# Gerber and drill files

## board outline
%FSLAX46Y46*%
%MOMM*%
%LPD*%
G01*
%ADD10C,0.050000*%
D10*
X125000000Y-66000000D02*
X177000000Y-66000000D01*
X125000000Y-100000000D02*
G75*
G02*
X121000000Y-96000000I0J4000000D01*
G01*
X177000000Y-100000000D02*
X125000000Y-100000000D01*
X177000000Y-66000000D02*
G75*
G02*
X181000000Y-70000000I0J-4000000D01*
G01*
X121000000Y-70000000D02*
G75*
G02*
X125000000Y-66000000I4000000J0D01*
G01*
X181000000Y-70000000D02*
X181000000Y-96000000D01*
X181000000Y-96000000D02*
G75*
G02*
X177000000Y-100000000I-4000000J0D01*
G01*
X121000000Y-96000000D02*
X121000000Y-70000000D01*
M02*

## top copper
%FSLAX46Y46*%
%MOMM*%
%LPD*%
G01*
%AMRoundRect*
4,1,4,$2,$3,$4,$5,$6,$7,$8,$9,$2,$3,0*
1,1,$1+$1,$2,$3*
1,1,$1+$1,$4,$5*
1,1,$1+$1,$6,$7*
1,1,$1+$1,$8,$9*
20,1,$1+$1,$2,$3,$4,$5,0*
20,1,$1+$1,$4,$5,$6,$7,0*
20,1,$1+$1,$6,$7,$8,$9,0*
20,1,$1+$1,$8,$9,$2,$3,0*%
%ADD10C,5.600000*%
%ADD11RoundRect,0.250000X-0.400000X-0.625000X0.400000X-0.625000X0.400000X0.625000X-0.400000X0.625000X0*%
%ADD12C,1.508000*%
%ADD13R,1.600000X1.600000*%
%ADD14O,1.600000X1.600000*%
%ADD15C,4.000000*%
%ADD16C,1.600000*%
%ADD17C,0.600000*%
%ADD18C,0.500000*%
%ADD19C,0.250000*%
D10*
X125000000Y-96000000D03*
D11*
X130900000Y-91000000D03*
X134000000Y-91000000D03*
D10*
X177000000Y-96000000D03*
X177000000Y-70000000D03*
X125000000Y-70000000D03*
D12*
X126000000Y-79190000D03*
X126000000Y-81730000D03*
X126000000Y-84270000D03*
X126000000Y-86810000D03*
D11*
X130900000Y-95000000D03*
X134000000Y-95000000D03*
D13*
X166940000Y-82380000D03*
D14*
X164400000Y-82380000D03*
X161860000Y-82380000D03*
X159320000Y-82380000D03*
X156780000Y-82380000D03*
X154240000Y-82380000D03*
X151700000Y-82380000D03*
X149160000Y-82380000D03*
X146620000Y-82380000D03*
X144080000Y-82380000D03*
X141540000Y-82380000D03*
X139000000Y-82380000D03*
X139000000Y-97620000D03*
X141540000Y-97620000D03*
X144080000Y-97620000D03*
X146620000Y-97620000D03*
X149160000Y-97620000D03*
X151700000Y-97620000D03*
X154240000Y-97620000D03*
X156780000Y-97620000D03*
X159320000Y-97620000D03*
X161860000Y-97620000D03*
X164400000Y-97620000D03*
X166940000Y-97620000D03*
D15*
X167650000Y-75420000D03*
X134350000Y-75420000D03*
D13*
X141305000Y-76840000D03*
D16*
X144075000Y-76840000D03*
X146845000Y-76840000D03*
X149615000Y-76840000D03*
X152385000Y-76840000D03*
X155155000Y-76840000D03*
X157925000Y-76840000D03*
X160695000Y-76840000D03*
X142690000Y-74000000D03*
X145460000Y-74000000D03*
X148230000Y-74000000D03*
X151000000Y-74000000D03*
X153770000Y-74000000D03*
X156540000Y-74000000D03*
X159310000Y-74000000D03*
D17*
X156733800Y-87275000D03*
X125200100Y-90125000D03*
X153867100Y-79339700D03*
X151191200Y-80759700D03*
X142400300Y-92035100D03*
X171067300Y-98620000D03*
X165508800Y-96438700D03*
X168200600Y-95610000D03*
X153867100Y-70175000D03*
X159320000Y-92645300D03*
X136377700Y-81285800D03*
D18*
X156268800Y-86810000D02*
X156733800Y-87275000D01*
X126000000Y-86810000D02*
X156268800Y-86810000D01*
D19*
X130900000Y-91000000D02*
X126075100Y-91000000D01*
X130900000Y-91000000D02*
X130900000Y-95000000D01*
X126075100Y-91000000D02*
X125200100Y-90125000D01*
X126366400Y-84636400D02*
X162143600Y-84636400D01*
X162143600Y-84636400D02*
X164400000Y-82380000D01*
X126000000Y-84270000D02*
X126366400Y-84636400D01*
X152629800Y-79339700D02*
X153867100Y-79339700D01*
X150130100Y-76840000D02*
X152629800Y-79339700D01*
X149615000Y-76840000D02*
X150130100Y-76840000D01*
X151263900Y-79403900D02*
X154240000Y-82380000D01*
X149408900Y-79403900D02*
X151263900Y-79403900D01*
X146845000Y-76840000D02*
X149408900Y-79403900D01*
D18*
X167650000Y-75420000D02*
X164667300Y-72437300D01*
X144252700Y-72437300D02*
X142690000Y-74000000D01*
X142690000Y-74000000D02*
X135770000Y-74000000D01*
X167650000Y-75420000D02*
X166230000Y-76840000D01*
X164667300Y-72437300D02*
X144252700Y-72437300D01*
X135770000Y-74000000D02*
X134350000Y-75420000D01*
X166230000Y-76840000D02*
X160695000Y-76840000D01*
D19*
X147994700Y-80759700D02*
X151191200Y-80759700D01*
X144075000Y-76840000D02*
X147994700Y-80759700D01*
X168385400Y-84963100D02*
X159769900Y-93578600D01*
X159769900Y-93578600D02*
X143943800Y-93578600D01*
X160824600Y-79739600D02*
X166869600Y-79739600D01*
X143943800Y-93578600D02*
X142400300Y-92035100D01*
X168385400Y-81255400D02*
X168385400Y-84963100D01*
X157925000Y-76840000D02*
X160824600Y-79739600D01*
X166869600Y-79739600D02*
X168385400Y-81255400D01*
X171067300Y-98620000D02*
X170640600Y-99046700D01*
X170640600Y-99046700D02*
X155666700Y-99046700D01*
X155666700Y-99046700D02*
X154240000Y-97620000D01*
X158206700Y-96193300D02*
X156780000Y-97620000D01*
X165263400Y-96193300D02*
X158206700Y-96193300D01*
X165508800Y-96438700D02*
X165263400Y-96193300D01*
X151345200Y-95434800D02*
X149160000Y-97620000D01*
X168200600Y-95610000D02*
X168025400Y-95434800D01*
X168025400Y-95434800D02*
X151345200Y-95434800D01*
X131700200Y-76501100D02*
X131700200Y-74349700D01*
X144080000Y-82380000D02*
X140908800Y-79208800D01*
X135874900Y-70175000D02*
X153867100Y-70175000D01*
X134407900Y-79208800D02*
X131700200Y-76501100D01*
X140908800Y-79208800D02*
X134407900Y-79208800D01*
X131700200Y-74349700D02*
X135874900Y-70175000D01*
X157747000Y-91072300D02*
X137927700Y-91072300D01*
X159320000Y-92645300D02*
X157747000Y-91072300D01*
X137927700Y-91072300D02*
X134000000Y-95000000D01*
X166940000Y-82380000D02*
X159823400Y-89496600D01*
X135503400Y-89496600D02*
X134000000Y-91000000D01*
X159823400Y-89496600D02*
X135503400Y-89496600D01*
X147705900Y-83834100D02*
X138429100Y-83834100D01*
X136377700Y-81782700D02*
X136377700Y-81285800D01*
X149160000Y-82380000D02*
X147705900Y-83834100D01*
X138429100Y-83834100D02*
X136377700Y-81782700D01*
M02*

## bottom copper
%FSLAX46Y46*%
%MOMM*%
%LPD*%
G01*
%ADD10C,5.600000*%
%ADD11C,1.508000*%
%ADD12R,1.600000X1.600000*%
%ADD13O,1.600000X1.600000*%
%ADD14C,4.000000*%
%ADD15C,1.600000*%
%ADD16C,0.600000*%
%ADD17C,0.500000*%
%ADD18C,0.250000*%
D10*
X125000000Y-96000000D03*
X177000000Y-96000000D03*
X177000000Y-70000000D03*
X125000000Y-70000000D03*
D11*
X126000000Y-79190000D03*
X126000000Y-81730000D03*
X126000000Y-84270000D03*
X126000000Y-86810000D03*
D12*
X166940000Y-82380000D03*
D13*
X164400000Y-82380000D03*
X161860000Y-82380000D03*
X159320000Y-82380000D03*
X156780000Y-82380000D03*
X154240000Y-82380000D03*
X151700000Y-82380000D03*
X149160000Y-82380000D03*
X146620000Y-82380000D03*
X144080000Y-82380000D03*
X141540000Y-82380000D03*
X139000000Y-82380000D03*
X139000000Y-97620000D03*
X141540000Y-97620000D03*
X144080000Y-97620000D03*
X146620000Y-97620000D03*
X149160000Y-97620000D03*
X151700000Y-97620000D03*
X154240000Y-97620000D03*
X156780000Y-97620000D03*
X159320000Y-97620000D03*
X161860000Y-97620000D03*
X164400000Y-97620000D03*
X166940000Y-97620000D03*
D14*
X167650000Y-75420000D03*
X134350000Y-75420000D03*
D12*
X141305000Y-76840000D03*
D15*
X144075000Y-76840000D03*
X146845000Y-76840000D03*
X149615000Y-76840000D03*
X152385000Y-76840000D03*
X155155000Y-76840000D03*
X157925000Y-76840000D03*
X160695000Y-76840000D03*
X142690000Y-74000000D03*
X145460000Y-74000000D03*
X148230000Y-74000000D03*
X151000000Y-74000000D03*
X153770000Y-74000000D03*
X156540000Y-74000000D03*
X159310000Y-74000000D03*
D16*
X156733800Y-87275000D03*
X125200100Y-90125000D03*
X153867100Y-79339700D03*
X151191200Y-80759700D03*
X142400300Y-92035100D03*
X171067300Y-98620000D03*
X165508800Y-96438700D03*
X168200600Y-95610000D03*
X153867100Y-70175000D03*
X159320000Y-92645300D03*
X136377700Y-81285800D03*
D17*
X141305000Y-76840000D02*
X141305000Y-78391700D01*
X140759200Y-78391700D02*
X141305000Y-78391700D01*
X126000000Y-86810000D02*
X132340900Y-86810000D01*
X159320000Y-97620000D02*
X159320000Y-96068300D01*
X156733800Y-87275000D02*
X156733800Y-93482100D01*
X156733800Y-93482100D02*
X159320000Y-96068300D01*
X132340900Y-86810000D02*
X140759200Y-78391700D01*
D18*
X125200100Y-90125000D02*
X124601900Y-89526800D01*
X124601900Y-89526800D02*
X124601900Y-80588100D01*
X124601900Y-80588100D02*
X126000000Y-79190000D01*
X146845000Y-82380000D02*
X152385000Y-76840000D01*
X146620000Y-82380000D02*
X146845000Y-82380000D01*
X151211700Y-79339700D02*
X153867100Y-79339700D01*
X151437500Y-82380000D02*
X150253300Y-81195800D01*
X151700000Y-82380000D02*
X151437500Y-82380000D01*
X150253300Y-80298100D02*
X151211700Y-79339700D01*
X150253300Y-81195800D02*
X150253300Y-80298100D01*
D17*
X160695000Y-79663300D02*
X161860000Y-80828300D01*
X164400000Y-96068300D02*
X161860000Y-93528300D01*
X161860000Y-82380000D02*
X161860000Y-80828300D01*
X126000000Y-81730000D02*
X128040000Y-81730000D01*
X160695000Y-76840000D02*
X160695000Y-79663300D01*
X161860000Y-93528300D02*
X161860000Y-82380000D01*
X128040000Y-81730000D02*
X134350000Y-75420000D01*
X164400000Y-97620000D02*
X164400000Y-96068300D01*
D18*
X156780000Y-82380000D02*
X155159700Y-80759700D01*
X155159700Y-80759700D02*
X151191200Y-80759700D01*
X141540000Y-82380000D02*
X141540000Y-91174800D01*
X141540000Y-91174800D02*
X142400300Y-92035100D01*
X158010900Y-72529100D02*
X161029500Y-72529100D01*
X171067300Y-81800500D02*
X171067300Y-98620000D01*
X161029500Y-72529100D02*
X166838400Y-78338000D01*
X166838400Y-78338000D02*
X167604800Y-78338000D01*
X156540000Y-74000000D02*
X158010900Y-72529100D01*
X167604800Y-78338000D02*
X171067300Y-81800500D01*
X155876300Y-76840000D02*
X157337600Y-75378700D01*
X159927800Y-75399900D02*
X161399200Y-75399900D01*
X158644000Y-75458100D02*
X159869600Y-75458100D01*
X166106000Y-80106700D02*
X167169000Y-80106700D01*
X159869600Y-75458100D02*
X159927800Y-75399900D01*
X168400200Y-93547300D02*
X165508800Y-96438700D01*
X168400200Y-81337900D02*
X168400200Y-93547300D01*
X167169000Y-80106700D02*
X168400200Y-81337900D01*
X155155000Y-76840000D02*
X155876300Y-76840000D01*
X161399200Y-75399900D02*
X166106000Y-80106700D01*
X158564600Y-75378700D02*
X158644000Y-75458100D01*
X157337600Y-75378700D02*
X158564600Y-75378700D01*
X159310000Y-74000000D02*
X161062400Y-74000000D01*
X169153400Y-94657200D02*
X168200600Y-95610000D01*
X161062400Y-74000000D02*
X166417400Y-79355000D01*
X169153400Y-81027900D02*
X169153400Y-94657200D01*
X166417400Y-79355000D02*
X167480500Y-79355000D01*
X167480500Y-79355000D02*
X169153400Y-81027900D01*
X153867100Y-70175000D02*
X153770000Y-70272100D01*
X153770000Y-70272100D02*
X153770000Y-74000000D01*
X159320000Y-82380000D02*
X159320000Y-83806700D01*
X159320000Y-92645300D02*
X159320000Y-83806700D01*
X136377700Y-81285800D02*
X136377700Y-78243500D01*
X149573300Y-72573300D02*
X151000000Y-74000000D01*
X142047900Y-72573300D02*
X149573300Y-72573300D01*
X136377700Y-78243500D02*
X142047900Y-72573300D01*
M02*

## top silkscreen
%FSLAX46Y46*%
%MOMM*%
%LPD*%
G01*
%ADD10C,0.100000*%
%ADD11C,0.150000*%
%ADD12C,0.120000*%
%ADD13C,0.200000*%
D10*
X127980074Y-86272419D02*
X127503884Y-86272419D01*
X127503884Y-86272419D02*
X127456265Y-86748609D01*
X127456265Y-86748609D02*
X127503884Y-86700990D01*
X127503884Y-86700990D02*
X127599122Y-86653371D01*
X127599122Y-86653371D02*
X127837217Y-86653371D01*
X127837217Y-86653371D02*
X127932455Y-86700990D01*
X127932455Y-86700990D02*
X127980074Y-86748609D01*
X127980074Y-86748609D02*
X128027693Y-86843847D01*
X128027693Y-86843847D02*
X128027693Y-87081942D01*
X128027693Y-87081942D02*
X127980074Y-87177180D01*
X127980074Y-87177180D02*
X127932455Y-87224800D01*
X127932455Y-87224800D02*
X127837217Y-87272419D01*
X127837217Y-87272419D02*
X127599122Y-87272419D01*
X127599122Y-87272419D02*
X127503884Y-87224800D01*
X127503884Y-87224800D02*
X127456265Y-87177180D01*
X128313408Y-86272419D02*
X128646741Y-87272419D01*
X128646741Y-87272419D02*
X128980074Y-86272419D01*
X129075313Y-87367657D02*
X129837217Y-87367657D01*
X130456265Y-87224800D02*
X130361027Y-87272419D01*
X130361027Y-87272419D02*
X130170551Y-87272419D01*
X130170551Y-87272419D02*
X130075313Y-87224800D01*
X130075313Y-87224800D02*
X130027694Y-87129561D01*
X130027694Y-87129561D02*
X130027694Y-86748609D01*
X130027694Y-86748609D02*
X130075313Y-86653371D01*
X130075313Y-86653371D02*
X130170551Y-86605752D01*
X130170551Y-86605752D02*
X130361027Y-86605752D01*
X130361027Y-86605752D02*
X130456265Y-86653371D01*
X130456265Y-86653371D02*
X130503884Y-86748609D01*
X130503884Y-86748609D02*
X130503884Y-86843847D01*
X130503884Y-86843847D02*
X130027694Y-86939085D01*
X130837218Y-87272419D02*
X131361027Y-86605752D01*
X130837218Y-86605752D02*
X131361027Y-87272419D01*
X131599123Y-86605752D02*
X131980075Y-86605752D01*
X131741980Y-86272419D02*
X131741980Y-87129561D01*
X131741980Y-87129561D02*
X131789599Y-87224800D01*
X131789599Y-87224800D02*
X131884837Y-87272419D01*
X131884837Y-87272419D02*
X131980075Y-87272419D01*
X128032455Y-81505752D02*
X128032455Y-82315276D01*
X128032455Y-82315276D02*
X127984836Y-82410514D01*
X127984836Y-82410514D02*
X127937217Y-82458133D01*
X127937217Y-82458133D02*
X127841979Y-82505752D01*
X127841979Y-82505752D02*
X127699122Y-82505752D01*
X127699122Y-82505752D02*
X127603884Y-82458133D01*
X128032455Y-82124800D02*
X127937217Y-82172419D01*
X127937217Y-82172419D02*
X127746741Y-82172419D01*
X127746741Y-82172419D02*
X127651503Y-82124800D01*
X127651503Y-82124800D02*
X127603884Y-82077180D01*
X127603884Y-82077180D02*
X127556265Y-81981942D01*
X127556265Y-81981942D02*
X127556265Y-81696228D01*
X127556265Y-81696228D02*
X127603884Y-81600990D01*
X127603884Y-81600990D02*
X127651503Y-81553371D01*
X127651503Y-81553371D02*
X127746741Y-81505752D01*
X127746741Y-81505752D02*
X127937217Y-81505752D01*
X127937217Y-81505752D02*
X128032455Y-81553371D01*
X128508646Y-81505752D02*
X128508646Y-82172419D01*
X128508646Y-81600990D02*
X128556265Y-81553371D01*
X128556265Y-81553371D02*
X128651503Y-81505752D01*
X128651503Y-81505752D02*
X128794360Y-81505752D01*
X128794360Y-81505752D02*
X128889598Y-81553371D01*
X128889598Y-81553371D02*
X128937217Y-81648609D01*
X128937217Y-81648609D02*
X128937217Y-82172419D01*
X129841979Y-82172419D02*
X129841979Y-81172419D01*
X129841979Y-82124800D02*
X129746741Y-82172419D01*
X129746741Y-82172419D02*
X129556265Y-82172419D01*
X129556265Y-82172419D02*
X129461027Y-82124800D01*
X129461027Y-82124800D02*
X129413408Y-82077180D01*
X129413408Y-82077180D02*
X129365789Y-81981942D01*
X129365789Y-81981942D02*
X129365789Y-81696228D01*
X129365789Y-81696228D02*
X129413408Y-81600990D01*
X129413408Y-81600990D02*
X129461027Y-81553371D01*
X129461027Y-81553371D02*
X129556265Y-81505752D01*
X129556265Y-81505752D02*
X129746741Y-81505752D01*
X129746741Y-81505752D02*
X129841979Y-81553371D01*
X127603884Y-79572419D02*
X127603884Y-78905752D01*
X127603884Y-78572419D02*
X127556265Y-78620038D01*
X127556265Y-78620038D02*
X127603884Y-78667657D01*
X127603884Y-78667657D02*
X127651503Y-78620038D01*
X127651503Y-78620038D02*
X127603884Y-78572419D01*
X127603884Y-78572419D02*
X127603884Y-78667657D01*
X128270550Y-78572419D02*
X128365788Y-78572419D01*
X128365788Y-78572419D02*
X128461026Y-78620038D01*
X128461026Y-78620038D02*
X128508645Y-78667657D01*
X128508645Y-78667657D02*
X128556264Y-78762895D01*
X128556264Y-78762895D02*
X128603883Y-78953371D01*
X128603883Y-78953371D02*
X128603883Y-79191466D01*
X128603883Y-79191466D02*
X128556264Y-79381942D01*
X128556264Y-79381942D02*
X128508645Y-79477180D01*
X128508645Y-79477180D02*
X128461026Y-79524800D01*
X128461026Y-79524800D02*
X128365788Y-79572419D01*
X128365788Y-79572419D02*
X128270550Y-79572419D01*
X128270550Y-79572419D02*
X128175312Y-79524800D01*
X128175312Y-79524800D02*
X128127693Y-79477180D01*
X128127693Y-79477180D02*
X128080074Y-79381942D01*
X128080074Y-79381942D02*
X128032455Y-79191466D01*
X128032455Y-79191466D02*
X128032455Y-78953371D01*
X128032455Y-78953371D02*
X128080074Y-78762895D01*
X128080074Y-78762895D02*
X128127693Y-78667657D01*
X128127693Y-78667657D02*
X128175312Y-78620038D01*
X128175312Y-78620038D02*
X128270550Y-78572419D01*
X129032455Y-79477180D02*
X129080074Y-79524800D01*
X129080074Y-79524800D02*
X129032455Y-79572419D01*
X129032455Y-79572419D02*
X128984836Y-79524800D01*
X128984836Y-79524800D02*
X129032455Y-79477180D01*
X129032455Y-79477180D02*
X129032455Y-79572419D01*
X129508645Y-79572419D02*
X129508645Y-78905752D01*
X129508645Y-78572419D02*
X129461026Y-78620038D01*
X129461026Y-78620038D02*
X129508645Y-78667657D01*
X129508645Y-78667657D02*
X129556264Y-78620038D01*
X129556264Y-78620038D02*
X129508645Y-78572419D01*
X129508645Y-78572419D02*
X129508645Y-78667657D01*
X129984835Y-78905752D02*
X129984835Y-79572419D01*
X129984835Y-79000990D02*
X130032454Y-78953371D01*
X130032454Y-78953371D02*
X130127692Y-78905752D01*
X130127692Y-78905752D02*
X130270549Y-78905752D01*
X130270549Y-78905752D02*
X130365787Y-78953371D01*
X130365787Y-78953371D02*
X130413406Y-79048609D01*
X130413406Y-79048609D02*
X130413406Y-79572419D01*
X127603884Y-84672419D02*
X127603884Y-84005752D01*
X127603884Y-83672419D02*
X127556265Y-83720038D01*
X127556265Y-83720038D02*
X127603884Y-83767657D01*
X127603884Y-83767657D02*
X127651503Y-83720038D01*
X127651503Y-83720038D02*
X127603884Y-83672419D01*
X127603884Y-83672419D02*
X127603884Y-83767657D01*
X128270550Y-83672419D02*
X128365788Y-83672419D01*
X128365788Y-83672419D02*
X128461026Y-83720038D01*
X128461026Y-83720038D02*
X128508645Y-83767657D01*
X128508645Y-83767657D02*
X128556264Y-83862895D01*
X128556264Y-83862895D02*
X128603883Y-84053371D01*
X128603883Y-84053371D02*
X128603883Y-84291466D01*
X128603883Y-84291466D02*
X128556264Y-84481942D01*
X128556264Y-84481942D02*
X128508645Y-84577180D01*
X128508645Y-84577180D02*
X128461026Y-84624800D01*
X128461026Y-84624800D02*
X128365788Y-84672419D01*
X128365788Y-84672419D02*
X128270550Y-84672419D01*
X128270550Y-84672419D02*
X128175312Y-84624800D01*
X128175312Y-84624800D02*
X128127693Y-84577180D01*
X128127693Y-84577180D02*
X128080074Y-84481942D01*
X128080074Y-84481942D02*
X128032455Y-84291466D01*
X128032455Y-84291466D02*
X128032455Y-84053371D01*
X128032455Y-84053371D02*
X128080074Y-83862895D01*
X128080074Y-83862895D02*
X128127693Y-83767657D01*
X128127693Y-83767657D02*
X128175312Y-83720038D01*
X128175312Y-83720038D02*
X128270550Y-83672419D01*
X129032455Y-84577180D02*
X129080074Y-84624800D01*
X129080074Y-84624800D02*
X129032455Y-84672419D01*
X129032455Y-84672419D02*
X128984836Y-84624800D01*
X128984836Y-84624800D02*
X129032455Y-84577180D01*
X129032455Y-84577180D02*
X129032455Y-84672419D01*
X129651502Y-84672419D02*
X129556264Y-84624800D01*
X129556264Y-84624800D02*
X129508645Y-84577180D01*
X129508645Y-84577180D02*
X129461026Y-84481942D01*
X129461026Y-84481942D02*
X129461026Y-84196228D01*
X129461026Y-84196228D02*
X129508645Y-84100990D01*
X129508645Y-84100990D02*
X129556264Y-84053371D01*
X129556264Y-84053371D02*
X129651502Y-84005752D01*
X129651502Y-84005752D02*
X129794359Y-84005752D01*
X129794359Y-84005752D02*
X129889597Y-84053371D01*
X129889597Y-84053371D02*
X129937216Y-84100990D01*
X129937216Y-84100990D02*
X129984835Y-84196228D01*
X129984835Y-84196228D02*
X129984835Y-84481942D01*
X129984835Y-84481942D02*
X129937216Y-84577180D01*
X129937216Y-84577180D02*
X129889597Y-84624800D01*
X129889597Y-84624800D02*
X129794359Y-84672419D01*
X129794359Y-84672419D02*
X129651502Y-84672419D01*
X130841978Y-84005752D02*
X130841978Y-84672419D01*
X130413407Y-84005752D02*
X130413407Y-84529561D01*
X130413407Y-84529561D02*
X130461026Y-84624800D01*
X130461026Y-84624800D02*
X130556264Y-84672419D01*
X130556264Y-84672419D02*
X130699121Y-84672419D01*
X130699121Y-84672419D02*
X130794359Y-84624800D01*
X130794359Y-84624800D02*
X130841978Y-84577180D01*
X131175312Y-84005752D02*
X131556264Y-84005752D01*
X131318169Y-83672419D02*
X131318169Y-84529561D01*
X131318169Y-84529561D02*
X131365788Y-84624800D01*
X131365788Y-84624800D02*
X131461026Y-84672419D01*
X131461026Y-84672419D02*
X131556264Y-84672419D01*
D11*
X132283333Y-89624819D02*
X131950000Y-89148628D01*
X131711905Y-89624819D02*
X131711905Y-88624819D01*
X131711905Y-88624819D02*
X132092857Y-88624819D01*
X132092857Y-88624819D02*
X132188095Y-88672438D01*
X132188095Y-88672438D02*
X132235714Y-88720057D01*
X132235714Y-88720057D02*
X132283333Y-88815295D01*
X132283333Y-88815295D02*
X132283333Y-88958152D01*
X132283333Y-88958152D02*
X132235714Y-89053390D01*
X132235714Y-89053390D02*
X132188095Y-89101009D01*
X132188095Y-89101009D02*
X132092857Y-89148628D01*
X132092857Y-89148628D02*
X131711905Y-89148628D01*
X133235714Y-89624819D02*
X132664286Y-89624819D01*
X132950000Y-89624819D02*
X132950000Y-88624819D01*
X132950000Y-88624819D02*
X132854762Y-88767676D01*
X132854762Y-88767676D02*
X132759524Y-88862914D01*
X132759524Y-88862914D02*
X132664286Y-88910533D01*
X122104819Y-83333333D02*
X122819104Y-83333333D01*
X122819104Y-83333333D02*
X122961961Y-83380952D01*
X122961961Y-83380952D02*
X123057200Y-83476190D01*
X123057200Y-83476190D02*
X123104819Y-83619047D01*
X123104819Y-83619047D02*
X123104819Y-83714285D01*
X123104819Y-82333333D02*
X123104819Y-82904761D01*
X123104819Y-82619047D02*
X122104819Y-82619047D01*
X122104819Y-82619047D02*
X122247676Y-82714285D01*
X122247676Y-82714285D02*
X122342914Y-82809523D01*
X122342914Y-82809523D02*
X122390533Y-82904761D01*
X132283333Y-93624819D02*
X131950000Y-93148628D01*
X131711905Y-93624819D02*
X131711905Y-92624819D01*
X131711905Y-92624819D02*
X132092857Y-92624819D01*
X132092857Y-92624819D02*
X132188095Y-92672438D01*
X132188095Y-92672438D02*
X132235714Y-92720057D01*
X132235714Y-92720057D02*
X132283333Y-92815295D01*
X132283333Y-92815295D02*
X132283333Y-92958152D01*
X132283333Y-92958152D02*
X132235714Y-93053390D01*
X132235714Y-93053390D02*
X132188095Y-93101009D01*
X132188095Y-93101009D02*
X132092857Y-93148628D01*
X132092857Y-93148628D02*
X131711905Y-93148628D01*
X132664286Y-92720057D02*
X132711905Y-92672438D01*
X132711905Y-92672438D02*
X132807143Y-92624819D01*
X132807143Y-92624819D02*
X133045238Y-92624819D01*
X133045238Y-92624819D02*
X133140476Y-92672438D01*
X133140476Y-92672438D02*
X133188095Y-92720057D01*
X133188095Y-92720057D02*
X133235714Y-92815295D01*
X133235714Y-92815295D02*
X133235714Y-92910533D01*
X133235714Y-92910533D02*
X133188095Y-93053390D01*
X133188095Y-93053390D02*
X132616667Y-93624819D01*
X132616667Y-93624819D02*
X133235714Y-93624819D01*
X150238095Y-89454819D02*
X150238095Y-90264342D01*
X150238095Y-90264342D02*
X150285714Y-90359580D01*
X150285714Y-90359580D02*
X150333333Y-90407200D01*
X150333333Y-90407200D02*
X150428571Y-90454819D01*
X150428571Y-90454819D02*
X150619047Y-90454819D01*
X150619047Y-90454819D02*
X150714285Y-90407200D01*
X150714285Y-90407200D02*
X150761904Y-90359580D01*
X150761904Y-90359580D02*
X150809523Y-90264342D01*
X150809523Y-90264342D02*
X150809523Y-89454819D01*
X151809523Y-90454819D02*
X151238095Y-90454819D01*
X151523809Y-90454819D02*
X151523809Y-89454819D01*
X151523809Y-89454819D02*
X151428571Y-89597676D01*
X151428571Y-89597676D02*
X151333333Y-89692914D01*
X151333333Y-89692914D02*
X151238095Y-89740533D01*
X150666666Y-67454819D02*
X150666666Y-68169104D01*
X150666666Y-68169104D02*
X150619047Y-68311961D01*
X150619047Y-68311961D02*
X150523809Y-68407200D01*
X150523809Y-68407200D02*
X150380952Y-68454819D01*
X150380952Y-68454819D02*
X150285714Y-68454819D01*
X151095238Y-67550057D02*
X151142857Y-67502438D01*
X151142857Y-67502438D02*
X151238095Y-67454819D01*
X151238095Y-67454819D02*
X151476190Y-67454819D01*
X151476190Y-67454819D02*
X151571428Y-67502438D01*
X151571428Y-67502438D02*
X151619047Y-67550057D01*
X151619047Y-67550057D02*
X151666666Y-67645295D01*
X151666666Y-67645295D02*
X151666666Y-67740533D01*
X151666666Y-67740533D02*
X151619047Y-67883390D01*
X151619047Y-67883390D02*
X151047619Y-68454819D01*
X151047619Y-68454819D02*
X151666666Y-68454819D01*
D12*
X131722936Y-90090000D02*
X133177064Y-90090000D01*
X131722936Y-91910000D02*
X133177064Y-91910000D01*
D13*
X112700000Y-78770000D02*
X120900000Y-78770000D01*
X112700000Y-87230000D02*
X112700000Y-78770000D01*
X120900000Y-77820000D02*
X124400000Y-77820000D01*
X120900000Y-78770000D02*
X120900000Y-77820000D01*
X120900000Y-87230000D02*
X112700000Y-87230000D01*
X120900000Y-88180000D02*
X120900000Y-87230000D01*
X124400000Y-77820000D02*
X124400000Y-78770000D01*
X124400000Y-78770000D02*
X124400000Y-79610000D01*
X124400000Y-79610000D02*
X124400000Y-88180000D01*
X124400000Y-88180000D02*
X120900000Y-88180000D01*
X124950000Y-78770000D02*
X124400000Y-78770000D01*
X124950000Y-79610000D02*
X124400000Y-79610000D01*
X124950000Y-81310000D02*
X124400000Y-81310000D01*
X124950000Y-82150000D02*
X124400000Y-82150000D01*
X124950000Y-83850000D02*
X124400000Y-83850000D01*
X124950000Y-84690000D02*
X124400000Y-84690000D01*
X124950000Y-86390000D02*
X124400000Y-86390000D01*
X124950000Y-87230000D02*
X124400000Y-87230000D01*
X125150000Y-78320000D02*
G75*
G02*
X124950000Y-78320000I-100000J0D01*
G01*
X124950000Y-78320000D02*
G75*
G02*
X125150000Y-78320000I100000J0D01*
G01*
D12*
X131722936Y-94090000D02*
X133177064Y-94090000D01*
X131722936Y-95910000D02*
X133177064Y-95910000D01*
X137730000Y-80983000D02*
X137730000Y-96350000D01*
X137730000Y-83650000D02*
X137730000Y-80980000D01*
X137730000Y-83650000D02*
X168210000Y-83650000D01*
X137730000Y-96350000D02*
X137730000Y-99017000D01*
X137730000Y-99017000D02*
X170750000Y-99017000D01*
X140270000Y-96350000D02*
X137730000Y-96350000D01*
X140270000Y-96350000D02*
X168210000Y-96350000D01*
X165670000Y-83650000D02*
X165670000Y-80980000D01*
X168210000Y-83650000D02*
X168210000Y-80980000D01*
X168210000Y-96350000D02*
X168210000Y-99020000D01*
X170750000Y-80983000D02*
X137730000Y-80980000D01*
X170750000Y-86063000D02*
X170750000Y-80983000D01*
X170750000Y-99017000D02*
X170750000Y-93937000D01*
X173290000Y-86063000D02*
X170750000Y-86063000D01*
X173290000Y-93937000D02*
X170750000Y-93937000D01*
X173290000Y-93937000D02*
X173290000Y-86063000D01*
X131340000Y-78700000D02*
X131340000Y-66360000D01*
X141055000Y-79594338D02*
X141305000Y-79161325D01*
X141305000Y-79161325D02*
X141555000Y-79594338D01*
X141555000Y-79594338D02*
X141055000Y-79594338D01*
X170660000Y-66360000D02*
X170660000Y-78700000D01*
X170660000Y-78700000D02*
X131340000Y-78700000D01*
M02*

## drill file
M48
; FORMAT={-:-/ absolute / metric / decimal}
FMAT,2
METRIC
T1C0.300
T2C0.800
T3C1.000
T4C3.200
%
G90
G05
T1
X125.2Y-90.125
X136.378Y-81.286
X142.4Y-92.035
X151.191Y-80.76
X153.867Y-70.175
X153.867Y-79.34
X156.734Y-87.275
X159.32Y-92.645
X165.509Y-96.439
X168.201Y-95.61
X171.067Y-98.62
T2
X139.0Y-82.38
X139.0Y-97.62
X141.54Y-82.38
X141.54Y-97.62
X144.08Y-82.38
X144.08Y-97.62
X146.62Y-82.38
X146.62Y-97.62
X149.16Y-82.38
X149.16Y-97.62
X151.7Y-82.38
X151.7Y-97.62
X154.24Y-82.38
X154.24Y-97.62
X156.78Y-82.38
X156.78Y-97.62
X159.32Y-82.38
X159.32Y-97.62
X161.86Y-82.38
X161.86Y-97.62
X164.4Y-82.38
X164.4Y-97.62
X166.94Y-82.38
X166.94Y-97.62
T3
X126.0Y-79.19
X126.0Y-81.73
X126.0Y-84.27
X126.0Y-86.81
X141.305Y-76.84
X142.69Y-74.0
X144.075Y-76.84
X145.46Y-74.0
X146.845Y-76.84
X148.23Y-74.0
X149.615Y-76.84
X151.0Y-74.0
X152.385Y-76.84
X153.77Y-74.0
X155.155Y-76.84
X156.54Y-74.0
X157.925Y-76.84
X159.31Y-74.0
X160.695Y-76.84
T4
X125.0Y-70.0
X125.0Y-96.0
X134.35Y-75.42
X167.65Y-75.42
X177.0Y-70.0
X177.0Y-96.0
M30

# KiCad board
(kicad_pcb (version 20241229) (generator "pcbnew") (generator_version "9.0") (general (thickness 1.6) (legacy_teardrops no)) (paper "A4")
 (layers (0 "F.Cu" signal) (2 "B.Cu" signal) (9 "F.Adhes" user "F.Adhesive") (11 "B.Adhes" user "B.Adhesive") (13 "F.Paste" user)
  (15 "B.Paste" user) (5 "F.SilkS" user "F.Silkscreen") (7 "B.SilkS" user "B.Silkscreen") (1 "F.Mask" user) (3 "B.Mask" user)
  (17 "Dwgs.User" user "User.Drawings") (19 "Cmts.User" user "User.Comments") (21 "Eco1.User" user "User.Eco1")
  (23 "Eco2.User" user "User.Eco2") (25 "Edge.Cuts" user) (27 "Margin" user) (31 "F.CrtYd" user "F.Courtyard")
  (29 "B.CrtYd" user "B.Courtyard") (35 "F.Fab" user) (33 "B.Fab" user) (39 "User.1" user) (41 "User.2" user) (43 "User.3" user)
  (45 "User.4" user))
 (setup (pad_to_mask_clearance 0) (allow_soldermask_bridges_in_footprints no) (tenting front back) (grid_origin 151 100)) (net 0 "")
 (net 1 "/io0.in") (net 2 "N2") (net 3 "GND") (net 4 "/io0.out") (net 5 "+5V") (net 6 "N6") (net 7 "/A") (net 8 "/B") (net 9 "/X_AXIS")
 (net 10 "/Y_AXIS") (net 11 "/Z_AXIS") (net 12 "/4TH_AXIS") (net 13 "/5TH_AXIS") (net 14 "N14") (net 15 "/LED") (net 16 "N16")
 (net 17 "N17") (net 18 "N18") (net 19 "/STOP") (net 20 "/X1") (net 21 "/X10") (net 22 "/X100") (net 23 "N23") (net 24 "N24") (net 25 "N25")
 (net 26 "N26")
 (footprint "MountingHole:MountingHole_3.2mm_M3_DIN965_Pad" (layer "F.Cu") (at 125 96)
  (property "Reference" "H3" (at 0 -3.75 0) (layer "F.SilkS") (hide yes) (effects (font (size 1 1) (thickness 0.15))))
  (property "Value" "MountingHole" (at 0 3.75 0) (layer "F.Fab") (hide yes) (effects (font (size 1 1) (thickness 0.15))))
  (pad "1" thru_hole circle (at 0 0) (size 5.6 5.6) (drill 3.2) (layers "*.Cu" "*.Mask") (remove_unused_layers no) (zone_connect 2)))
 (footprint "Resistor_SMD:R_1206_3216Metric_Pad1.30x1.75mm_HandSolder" (layer "F.Cu") (at 132.45 91)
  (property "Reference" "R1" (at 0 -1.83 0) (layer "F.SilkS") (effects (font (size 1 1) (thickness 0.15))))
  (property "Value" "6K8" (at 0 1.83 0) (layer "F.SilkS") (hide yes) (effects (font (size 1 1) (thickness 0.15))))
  (fp_line (start -0.727064 -0.91) (end 0.727064 -0.91) (stroke (width 0.12) (type solid)) (layer "F.SilkS"))
  (fp_line (start -0.727064 0.91) (end 0.727064 0.91) (stroke (width 0.12) (type solid)) (layer "F.SilkS"))
  (pad "1" smd roundrect (at -1.55 0) (size 1.3 1.75) (layers "F.Cu" "F.Mask" "F.Paste") (roundrect_rratio 0.192308) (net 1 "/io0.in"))
  (pad "2" smd roundrect (at 1.55 0) (size 1.3 1.75) (layers "F.Cu" "F.Mask" "F.Paste") (roundrect_rratio 0.192308) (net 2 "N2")))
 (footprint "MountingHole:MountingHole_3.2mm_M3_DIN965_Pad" (layer "F.Cu") (at 177 96)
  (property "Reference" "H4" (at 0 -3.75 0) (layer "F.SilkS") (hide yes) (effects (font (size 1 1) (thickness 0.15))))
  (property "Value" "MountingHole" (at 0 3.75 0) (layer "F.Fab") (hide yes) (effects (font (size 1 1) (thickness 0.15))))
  (pad "1" thru_hole circle (at 0 0) (size 5.6 5.6) (drill 3.2) (layers "*.Cu" "*.Mask") (remove_unused_layers no) (zone_connect 2)))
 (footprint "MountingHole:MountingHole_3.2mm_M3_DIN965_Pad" (layer "F.Cu") (at 177 70)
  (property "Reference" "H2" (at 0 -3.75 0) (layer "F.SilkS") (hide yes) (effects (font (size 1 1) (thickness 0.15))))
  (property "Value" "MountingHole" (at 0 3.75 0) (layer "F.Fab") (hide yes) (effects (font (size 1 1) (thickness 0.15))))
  (pad "1" thru_hole circle (at 0 0) (size 5.6 5.6) (drill 3.2) (layers "*.Cu" "*.Mask") (remove_unused_layers no) (zone_connect 2)))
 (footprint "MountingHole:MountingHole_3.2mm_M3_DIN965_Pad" (layer "F.Cu") (at 125 70)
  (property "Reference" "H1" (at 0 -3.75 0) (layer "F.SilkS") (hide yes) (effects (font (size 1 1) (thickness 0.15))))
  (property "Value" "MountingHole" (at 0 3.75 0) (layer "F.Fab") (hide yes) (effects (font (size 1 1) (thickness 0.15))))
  (pad "1" thru_hole circle (at 0 0) (size 5.6 5.6) (drill 3.2) (layers "*.Cu" "*.Mask") (remove_unused_layers no) (zone_connect 2)))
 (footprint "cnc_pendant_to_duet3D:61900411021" (layer "F.Cu") (at 122.65 83 -90)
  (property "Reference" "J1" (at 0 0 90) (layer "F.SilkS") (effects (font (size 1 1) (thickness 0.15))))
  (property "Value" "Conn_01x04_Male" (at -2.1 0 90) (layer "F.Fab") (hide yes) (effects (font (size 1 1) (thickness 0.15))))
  (fp_line (start -4.23 9.95) (end -4.23 1.75) (stroke (width 0.2) (type solid)) (layer "F.SilkS"))
  (fp_line (start 4.23 9.95) (end -4.23 9.95) (stroke (width 0.2) (type solid)) (layer "F.SilkS"))
  (fp_line (start -5.18 1.75) (end -5.18 -1.75) (stroke (width 0.2) (type solid)) (layer "F.SilkS"))
  (fp_line (start -4.23 1.75) (end -5.18 1.75) (stroke (width 0.2) (type solid)) (layer "F.SilkS"))
  (fp_line (start 4.23 1.75) (end 4.23 9.95) (stroke (width 0.2) (type solid)) (layer "F.SilkS"))
  (fp_line (start 5.18 1.75) (end 4.23 1.75) (stroke (width 0.2) (type solid)) (layer "F.SilkS"))
  (fp_line (start -5.18 -1.75) (end -4.23 -1.75) (stroke (width 0.2) (type solid)) (layer "F.SilkS"))
  (fp_line (start -4.23 -1.75) (end -3.39 -1.75) (stroke (width 0.2) (type solid)) (layer "F.SilkS"))
  (fp_line (start -3.39 -1.75) (end 5.18 -1.75) (stroke (width 0.2) (type solid)) (layer "F.SilkS"))
  (fp_line (start 5.18 -1.75) (end 5.18 1.75) (stroke (width 0.2) (type solid)) (layer "F.SilkS"))
  (fp_line (start -4.23 -2.3) (end -4.23 -1.75) (stroke (width 0.2) (type solid)) (layer "F.SilkS"))
  (fp_line (start -3.39 -2.3) (end -3.39 -1.75) (stroke (width 0.2) (type solid)) (layer "F.SilkS"))
  (fp_line (start -1.69 -2.3) (end -1.69 -1.75) (stroke (width 0.2) (type solid)) (layer "F.SilkS"))
  (fp_line (start -0.85 -2.3) (end -0.85 -1.75) (stroke (width 0.2) (type solid)) (layer "F.SilkS"))
  (fp_line (start 0.85 -2.3) (end 0.85 -1.75) (stroke (width 0.2) (type solid)) (layer "F.SilkS"))
  (fp_line (start 1.69 -2.3) (end 1.69 -1.75) (stroke (width 0.2) (type solid)) (layer "F.SilkS"))
  (fp_line (start 3.39 -2.3) (end 3.39 -1.75) (stroke (width 0.2) (type solid)) (layer "F.SilkS"))
  (fp_line (start 4.23 -2.3) (end 4.23 -1.75) (stroke (width 0.2) (type solid)) (layer "F.SilkS"))
  (fp_circle (center -4.68 -2.4) (end -4.58 -2.4) (stroke (width 0.2) (type solid)) (fill no) (layer "F.SilkS"))
  (pad "1" thru_hole circle (at -3.81 -3.35 270) (size 1.508 1.508) (drill 1) (layers "*.Cu" "*.Mask") (remove_unused_layers no)
   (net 1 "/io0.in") (solder_mask_margin 0.102))
  (pad "2" thru_hole circle (at -1.27 -3.35 270) (size 1.508 1.508) (drill 1) (layers "*.Cu" "*.Mask") (remove_unused_layers no)
   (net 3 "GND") (solder_mask_margin 0.102))
  (pad "3" thru_hole circle (at 1.27 -3.35 270) (size 1.508 1.508) (drill 1) (layers "*.Cu" "*.Mask") (remove_unused_layers no)
   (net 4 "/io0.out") (solder_mask_margin 0.102))
  (pad "4" thru_hole circle (at 3.81 -3.35 270) (size 1.508 1.508) (drill 1) (layers "*.Cu" "*.Mask") (remove_unused_layers no)
   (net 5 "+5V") (solder_mask_margin 0.102)))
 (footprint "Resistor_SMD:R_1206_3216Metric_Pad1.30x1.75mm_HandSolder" (layer "F.Cu") (at 132.45 95)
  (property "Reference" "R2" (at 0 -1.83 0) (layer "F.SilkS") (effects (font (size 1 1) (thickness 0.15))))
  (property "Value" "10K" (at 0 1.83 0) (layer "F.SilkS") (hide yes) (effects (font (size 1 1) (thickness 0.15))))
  (fp_line (start -0.727064 -0.91) (end 0.727064 -0.91) (stroke (width 0.12) (type solid)) (layer "F.SilkS"))
  (fp_line (start -0.727064 0.91) (end 0.727064 0.91) (stroke (width 0.12) (type solid)) (layer "F.SilkS"))
  (pad "1" smd roundrect (at -1.55 0) (size 1.3 1.75) (layers "F.Cu" "F.Mask" "F.Paste") (roundrect_rratio 0.192308) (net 1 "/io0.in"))
  (pad "2" smd roundrect (at 1.55 0) (size 1.3 1.75) (layers "F.Cu" "F.Mask" "F.Paste") (roundrect_rratio 0.192308) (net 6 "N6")))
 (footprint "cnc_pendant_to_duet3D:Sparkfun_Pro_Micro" (layer "F.Cu") (at 139 97.62 90)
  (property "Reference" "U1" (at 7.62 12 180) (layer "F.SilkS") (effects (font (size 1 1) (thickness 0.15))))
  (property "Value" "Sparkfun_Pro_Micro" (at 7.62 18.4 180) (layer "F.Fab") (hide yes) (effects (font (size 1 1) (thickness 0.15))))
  (fp_line (start 16.637 -1.27) (end 1.27 -1.27) (stroke (width 0.12) (type solid)) (layer "F.SilkS"))
  (fp_line (start 13.97 -1.27) (end 16.64 -1.27) (stroke (width 0.12) (type solid)) (layer "F.SilkS"))
  (fp_line (start 13.97 -1.27) (end 13.97 29.21) (stroke (width 0.12) (type solid)) (layer "F.SilkS"))
  (fp_line (start 1.27 -1.27) (end -1.397 -1.27) (stroke (width 0.12) (type solid)) (layer "F.SilkS"))
  (fp_line (start -1.397 -1.27) (end -1.397 31.75) (stroke (width 0.12) (type solid)) (layer "F.SilkS"))
  (fp_line (start 1.27 1.27) (end 1.27 -1.27) (stroke (width 0.12) (type solid)) (layer "F.SilkS"))
  (fp_line (start 1.27 1.27) (end 1.27 29.21) (stroke (width 0.12) (type solid)) (layer "F.SilkS"))
  (fp_line (start 13.97 26.67) (end 16.64 26.67) (stroke (width 0.12) (type solid)) (layer "F.SilkS"))
  (fp_line (start 13.97 29.21) (end 16.64 29.21) (stroke (width 0.12) (type solid)) (layer "F.SilkS"))
  (fp_line (start 1.27 29.21) (end -1.4 29.21) (stroke (width 0.12) (type solid)) (layer "F.SilkS"))
  (fp_line (start 16.637 31.75) (end 16.64 -1.27) (stroke (width 0.12) (type solid)) (layer "F.SilkS"))
  (fp_line (start 11.557 31.75) (end 16.637 31.75) (stroke (width 0.12) (type solid)) (layer "F.SilkS"))
  (fp_line (start -1.397 31.75) (end 3.683 31.75) (stroke (width 0.12) (type solid)) (layer "F.SilkS"))
  (fp_line (start 11.557 34.29) (end 11.557 31.75) (stroke (width 0.12) (type solid)) (layer "F.SilkS"))
  (fp_line (start 3.683 34.29) (end 3.683 31.75) (stroke (width 0.12) (type solid)) (layer "F.SilkS"))
  (fp_line (start 3.683 34.29) (end 11.557 34.29) (stroke (width 0.12) (type solid)) (layer "F.SilkS"))
  (pad "1" thru_hole rect (at 15.24 27.94 90) (size 1.6 1.6) (drill 0.8) (layers "*.Cu" "*.Mask") (remove_unused_layers no) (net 2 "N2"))
  (pad "2" thru_hole oval (at 15.24 25.4 90) (size 1.6 1.6) (drill 0.8) (layers "*.Cu" "*.Mask") (remove_unused_layers no)
   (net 4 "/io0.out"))
  (pad "3" thru_hole oval (at 15.24 22.86 90) (size 1.6 1.6) (drill 0.8) (layers "*.Cu" "*.Mask") (remove_unused_layers no) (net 3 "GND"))
  (pad "4" thru_hole oval (at 15.24 20.32 90) (size 1.6 1.6) (drill 0.8) (layers "*.Cu" "*.Mask") (remove_unused_layers no) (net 6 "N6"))
  (pad "5" thru_hole oval (at 15.24 17.78 90) (size 1.6 1.6) (drill 0.8) (layers "*.Cu" "*.Mask") (remove_unused_layers no) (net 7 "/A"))
  (pad "6" thru_hole oval (at 15.24 15.24 90) (size 1.6 1.6) (drill 0.8) (layers "*.Cu" "*.Mask") (remove_unused_layers no) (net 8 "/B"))
  (pad "7" thru_hole oval (at 15.24 12.7 90) (size 1.6 1.6) (drill 0.8) (layers "*.Cu" "*.Mask") (remove_unused_layers no) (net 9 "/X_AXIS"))
  (pad "8" thru_hole oval (at 15.24 10.16 90) (size 1.6 1.6) (drill 0.8) (layers "*.Cu" "*.Mask") (remove_unused_layers no)
   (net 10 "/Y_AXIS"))
  (pad "9" thru_hole oval (at 15.24 7.62 90) (size 1.6 1.6) (drill 0.8) (layers "*.Cu" "*.Mask") (remove_unused_layers no)
   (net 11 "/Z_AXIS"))
  (pad "10" thru_hole oval (at 15.24 5.08 90) (size 1.6 1.6) (drill 0.8) (layers "*.Cu" "*.Mask") (remove_unused_layers no)
   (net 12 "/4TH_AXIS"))
  (pad "11" thru_hole oval (at 15.24 2.54 90) (size 1.6 1.6) (drill 0.8) (layers "*.Cu" "*.Mask") (remove_unused_layers no)
   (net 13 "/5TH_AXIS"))
  (pad "12" thru_hole oval (at 15.24 0 90) (size 1.6 1.6) (drill 0.8) (layers "*.Cu" "*.Mask") (remove_unused_layers no) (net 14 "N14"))
  (pad "13" thru_hole oval (at 0 0 90) (size 1.6 1.6) (drill 0.8) (layers "*.Cu" "*.Mask") (remove_unused_layers no) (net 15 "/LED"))
  (pad "14" thru_hole oval (at 0 2.54 90) (size 1.6 1.6) (drill 0.8) (layers "*.Cu" "*.Mask") (remove_unused_layers no) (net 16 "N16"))
  (pad "15" thru_hole oval (at 0 5.08 90) (size 1.6 1.6) (drill 0.8) (layers "*.Cu" "*.Mask") (remove_unused_layers no) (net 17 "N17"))
  (pad "16" thru_hole oval (at 0 7.62 90) (size 1.6 1.6) (drill 0.8) (layers "*.Cu" "*.Mask") (remove_unused_layers no) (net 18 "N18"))
  (pad "17" thru_hole oval (at 0 10.16 90) (size 1.6 1.6) (drill 0.8) (layers "*.Cu" "*.Mask") (remove_unused_layers no) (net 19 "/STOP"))
  (pad "18" thru_hole oval (at 0 12.7 90) (size 1.6 1.6) (drill 0.8) (layers "*.Cu" "*.Mask") (remove_unused_layers no) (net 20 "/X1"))
  (pad "19" thru_hole oval (at 0 15.24 90) (size 1.6 1.6) (drill 0.8) (layers "*.Cu" "*.Mask") (remove_unused_layers no) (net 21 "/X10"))
  (pad "20" thru_hole oval (at 0 17.78 90) (size 1.6 1.6) (drill 0.8) (layers "*.Cu" "*.Mask") (remove_unused_layers no) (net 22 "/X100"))
  (pad "21" thru_hole oval (at 0 20.32 90) (size 1.6 1.6) (drill 0.8) (layers "*.Cu" "*.Mask") (remove_unused_layers no) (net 5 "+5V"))
  (pad "22" thru_hole oval (at 0 22.86 90) (size 1.6 1.6) (drill 0.8) (layers "*.Cu" "*.Mask") (remove_unused_layers no) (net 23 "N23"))
  (pad "23" thru_hole oval (at 0 25.4 90) (size 1.6 1.6) (drill 0.8) (layers "*.Cu" "*.Mask") (remove_unused_layers no) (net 3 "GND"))
  (pad "24" thru_hole oval (at 0 27.94 90) (size 1.6 1.6) (drill 0.8) (layers "*.Cu" "*.Mask") (remove_unused_layers no) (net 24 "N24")))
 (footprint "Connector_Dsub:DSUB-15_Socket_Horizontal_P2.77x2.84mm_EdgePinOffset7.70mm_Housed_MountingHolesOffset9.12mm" (layer "F.Cu")
  (at 141.305 76.84 180)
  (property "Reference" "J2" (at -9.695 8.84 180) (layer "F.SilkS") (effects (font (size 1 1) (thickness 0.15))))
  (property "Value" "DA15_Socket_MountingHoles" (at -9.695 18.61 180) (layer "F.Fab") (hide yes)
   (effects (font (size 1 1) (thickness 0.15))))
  (fp_line (start 9.965 -1.86) (end 9.965 10.48) (stroke (width 0.12) (type solid)) (layer "F.SilkS"))
  (fp_line (start 0.25 -2.754338) (end 0 -2.321325) (stroke (width 0.12) (type solid)) (layer "F.SilkS"))
  (fp_line (start 0 -2.321325) (end -0.25 -2.754338) (stroke (width 0.12) (type solid)) (layer "F.SilkS"))
  (fp_line (start -0.25 -2.754338) (end 0.25 -2.754338) (stroke (width 0.12) (type solid)) (layer "F.SilkS"))
  (fp_line (start -29.355 10.48) (end -29.355 -1.86) (stroke (width 0.12) (type solid)) (layer "F.SilkS"))
  (fp_line (start -29.355 -1.86) (end 9.965 -1.86) (stroke (width 0.12) (type solid)) (layer "F.SilkS"))
  (pad "0" thru_hole circle (at -26.345 1.42 180) (size 4 4) (drill 3.2) (layers "*.Cu" "*.Mask") (remove_unused_layers no) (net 3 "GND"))
  (pad "0" thru_hole circle (at 6.955 1.42 180) (size 4 4) (drill 3.2) (layers "*.Cu" "*.Mask") (remove_unused_layers no) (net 3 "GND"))
  (pad "1" thru_hole rect (at 0 0 180) (size 1.6 1.6) (drill 1) (layers "*.Cu" "*.Mask") (remove_unused_layers no) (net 5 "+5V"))
  (pad "2" thru_hole circle (at -2.77 0 180) (size 1.6 1.6) (drill 1) (layers "*.Cu" "*.Mask") (remove_unused_layers no) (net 7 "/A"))
  (pad "3" thru_hole circle (at -5.54 0 180) (size 1.6 1.6) (drill 1) (layers "*.Cu" "*.Mask") (remove_unused_layers no) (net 8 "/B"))
  (pad "4" thru_hole circle (at -8.31 0 180) (size 1.6 1.6) (drill 1) (layers "*.Cu" "*.Mask") (remove_unused_layers no) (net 9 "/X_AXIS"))
  (pad "5" thru_hole circle (at -11.08 0 180) (size 1.6 1.6) (drill 1) (layers "*.Cu" "*.Mask") (remove_unused_layers no) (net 11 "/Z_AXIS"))
  (pad "6" thru_hole circle (at -13.85 0 180) (size 1.6 1.6) (drill 1) (layers "*.Cu" "*.Mask") (remove_unused_layers no) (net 22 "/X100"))
  (pad "7" thru_hole circle (at -16.62 0 180) (size 1.6 1.6) (drill 1) (layers "*.Cu" "*.Mask") (remove_unused_layers no)
   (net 13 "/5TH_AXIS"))
  (pad "8" thru_hole circle (at -19.39 0 180) (size 1.6 1.6) (drill 1) (layers "*.Cu" "*.Mask") (remove_unused_layers no) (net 3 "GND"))
  (pad "9" thru_hole circle (at -1.385 2.84 180) (size 1.6 1.6) (drill 1) (layers "*.Cu" "*.Mask") (remove_unused_layers no) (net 3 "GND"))
  (pad "10" thru_hole circle (at -4.155 2.84 180) (size 1.6 1.6) (drill 1) (layers "*.Cu" "*.Mask") (remove_unused_layers no) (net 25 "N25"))
  (pad "11" thru_hole circle (at -6.925 2.84 180) (size 1.6 1.6) (drill 1) (layers "*.Cu" "*.Mask") (remove_unused_layers no) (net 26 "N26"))
  (pad "12" thru_hole circle (at -9.695 2.84 180) (size 1.6 1.6) (drill 1) (layers "*.Cu" "*.Mask") (remove_unused_layers no)
   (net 10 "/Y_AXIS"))
  (pad "13" thru_hole circle (at -12.465 2.84 180) (size 1.6 1.6) (drill 1) (layers "*.Cu" "*.Mask") (remove_unused_layers no)
   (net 12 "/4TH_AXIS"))
  (pad "14" thru_hole circle (at -15.235 2.84 180) (size 1.6 1.6) (drill 1) (layers "*.Cu" "*.Mask") (remove_unused_layers no)
   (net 21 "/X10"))
  (pad "15" thru_hole circle (at -18.005 2.84 180) (size 1.6 1.6) (drill 1) (layers "*.Cu" "*.Mask") (remove_unused_layers no)
   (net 19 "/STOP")))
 (gr_line (start 125 66) (end 177 66) (stroke (width 0.05) (type default)) (layer "Edge.Cuts"))
 (gr_arc (start 125 100) (mid 122.171573 98.828427) (end 121 96) (stroke (width 0.05) (type default)) (layer "Edge.Cuts"))
 (gr_line (start 177 100) (end 125 100) (stroke (width 0.05) (type default)) (layer "Edge.Cuts"))
 (gr_arc (start 177 66) (mid 179.828427 67.171573) (end 181 70) (stroke (width 0.05) (type default)) (layer "Edge.Cuts"))
 (gr_arc (start 121 70) (mid 122.171573 67.171573) (end 125 66) (stroke (width 0.05) (type default)) (layer "Edge.Cuts"))
 (gr_line (start 181 70) (end 181 96) (stroke (width 0.05) (type default)) (layer "Edge.Cuts"))
 (gr_arc (start 181 96) (mid 179.828427 98.828427) (end 177 100) (stroke (width 0.05) (type default)) (layer "Edge.Cuts"))
 (gr_line (start 121 96) (end 121 70) (stroke (width 0.05) (type default)) (layer "Edge.Cuts"))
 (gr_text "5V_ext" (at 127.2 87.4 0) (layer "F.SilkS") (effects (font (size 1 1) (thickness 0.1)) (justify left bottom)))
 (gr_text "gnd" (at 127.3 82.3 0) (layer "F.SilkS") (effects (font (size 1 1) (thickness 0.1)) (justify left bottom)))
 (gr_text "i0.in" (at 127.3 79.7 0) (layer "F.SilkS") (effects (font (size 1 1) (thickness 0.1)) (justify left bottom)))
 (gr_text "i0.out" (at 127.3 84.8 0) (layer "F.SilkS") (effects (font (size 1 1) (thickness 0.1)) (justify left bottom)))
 (segment (start 156.2688 86.81) (end 156.7338 87.275) (width 0.5) (layer "F.Cu") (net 5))
 (segment (start 126 86.81) (end 156.2688 86.81) (width 0.5) (layer "F.Cu") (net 5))
 (via (at 156.7338 87.275) (size 0.6) (drill 0.3) (layers "F.Cu" "B.Cu") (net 5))
 (segment (start 141.305 76.84) (end 141.305 78.3917) (width 0.5) (layer "B.Cu") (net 5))
 (segment (start 140.7592 78.3917) (end 141.305 78.3917) (width 0.5) (layer "B.Cu") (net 5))
 (segment (start 126 86.81) (end 132.3409 86.81) (width 0.5) (layer "B.Cu") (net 5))
 (segment (start 159.32 97.62) (end 159.32 96.0683) (width 0.5) (layer "B.Cu") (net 5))
 (segment (start 156.7338 87.275) (end 156.7338 93.4821) (width 0.5) (layer "B.Cu") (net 5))
 (segment (start 156.7338 93.4821) (end 159.32 96.0683) (width 0.5) (layer "B.Cu") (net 5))
 (segment (start 132.3409 86.81) (end 140.7592 78.3917) (width 0.5) (layer "B.Cu") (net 5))
 (segment (start 130.9 91) (end 126.0751 91) (width 0.25) (layer "F.Cu") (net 1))
 (segment (start 130.9 91) (end 130.9 95) (width 0.25) (layer "F.Cu") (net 1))
 (segment (start 126.0751 91) (end 125.2001 90.125) (width 0.25) (layer "F.Cu") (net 1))
 (via (at 125.2001 90.125) (size 0.6) (drill 0.3) (layers "F.Cu" "B.Cu") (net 1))
 (segment (start 125.2001 90.125) (end 124.6019 89.5268) (width 0.25) (layer "B.Cu") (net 1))
 (segment (start 124.6019 89.5268) (end 124.6019 80.5881) (width 0.25) (layer "B.Cu") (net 1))
 (segment (start 124.6019 80.5881) (end 126 79.19) (width 0.25) (layer "B.Cu") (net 1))
 (segment (start 126.3664 84.6364) (end 162.1436 84.6364) (width 0.25) (layer "F.Cu") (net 4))
 (segment (start 162.1436 84.6364) (end 164.4 82.38) (width 0.25) (layer "F.Cu") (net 4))
 (segment (start 126 84.27) (end 126.3664 84.6364) (width 0.25) (layer "F.Cu") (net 4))
 (segment (start 146.845 82.38) (end 152.385 76.84) (width 0.25) (layer "B.Cu") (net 11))
 (segment (start 146.62 82.38) (end 146.845 82.38) (width 0.25) (layer "B.Cu") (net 11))
 (segment (start 152.6298 79.3397) (end 153.8671 79.3397) (width 0.25) (layer "F.Cu") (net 9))
 (segment (start 150.1301 76.84) (end 152.6298 79.3397) (width 0.25) (layer "F.Cu") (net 9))
 (segment (start 149.615 76.84) (end 150.1301 76.84) (width 0.25) (layer "F.Cu") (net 9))
 (via (at 153.8671 79.3397) (size 0.6) (drill 0.3) (layers "F.Cu" "B.Cu") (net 9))
 (segment (start 151.2117 79.3397) (end 153.8671 79.3397) (width 0.25) (layer "B.Cu") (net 9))
 (segment (start 151.4375 82.38) (end 150.2533 81.1958) (width 0.25) (layer "B.Cu") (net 9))
 (segment (start 151.7 82.38) (end 151.4375 82.38) (width 0.25) (layer "B.Cu") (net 9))
 (segment (start 150.2533 80.2981) (end 151.2117 79.3397) (width 0.25) (layer "B.Cu") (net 9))
 (segment (start 150.2533 81.1958) (end 150.2533 80.2981) (width 0.25) (layer "B.Cu") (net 9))
 (segment (start 151.2639 79.4039) (end 154.24 82.38) (width 0.25) (layer "F.Cu") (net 8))
 (segment (start 149.4089 79.4039) (end 151.2639 79.4039) (width 0.25) (layer "F.Cu") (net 8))
 (segment (start 146.845 76.84) (end 149.4089 79.4039) (width 0.25) (layer "F.Cu") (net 8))
 (segment (start 167.65 75.42) (end 164.6673 72.4373) (width 0.5) (layer "F.Cu") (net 3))
 (segment (start 144.2527 72.4373) (end 142.69 74) (width 0.5) (layer "F.Cu") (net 3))
 (segment (start 142.69 74) (end 135.77 74) (width 0.5) (layer "F.Cu") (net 3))
 (segment (start 167.65 75.42) (end 166.23 76.84) (width 0.5) (layer "F.Cu") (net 3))
 (segment (start 164.6673 72.4373) (end 144.2527 72.4373) (width 0.5) (layer "F.Cu") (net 3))
 (segment (start 135.77 74) (end 134.35 75.42) (width 0.5) (layer "F.Cu") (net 3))
 (segment (start 166.23 76.84) (end 160.695 76.84) (width 0.5) (layer "F.Cu") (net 3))
 (segment (start 160.695 79.6633) (end 161.86 80.8283) (width 0.5) (layer "B.Cu") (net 3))
 (segment (start 164.4 96.0683) (end 161.86 93.5283) (width 0.5) (layer "B.Cu") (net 3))
 (segment (start 161.86 82.38) (end 161.86 80.8283) (width 0.5) (layer "B.Cu") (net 3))
 (segment (start 126 81.73) (end 128.04 81.73) (width 0.5) (layer "B.Cu") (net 3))
 (segment (start 160.695 76.84) (end 160.695 79.6633) (width 0.5) (layer "B.Cu") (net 3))
 (segment (start 161.86 93.5283) (end 161.86 82.38) (width 0.5) (layer "B.Cu") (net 3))
 (segment (start 128.04 81.73) (end 134.35 75.42) (width 0.5) (layer "B.Cu") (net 3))
 (segment (start 164.4 97.62) (end 164.4 96.0683) (width 0.5) (layer "B.Cu") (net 3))
 (segment (start 147.9947 80.7597) (end 151.1912 80.7597) (width 0.25) (layer "F.Cu") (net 7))
 (segment (start 144.075 76.84) (end 147.9947 80.7597) (width 0.25) (layer "F.Cu") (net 7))
 (via (at 151.1912 80.7597) (size 0.6) (drill 0.3) (layers "F.Cu" "B.Cu") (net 7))
 (segment (start 156.78 82.38) (end 155.1597 80.7597) (width 0.25) (layer "B.Cu") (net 7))
 (segment (start 155.1597 80.7597) (end 151.1912 80.7597) (width 0.25) (layer "B.Cu") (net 7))
 (segment (start 168.3854 84.9631) (end 159.7699 93.5786) (width 0.25) (layer "F.Cu") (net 13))
 (segment (start 159.7699 93.5786) (end 143.9438 93.5786) (width 0.25) (layer "F.Cu") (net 13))
 (segment (start 160.8246 79.7396) (end 166.8696 79.7396) (width 0.25) (layer "F.Cu") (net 13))
 (segment (start 143.9438 93.5786) (end 142.4003 92.0351) (width 0.25) (layer "F.Cu") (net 13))
 (segment (start 168.3854 81.2554) (end 168.3854 84.9631) (width 0.25) (layer "F.Cu") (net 13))
 (segment (start 157.925 76.84) (end 160.8246 79.7396) (width 0.25) (layer "F.Cu") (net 13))
 (segment (start 166.8696 79.7396) (end 168.3854 81.2554) (width 0.25) (layer "F.Cu") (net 13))
 (via (at 142.4003 92.0351) (size 0.6) (drill 0.3) (layers "F.Cu" "B.Cu") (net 13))
 (segment (start 141.54 82.38) (end 141.54 91.1748) (width 0.25) (layer "B.Cu") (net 13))
 (segment (start 141.54 91.1748) (end 142.4003 92.0351) (width 0.25) (layer "B.Cu") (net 13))
 (segment (start 171.0673 98.62) (end 170.6406 99.0467) (width 0.25) (layer "F.Cu") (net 21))
 (segment (start 170.6406 99.0467) (end 155.6667 99.0467) (width 0.25) (layer "F.Cu") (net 21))
 (segment (start 155.6667 99.0467) (end 154.24 97.62) (width 0.25) (layer "F.Cu") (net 21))
 (via (at 171.0673 98.62) (size 0.6) (drill 0.3) (layers "F.Cu" "B.Cu") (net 21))
 (segment (start 158.0109 72.5291) (end 161.0295 72.5291) (width 0.25) (layer "B.Cu") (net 21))
 (segment (start 171.0673 81.8005) (end 171.0673 98.62) (width 0.25) (layer "B.Cu") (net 21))
 (segment (start 161.0295 72.5291) (end 166.8384 78.338) (width 0.25) (layer "B.Cu") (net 21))
 (segment (start 166.8384 78.338) (end 167.6048 78.338) (width 0.25) (layer "B.Cu") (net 21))
 (segment (start 156.54 74) (end 158.0109 72.5291) (width 0.25) (layer "B.Cu") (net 21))
 (segment (start 167.6048 78.338) (end 171.0673 81.8005) (width 0.25) (layer "B.Cu") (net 21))
 (segment (start 158.2067 96.1933) (end 156.78 97.62) (width 0.25) (layer "F.Cu") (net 22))
 (segment (start 165.2634 96.1933) (end 158.2067 96.1933) (width 0.25) (layer "F.Cu") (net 22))
 (segment (start 165.5088 96.4387) (end 165.2634 96.1933) (width 0.25) (layer "F.Cu") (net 22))
 (via (at 165.5088 96.4387) (size 0.6) (drill 0.3) (layers "F.Cu" "B.Cu") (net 22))
 (segment (start 155.8763 76.84) (end 157.3376 75.3787) (width 0.25) (layer "B.Cu") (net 22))
 (segment (start 159.9278 75.3999) (end 161.3992 75.3999) (width 0.25) (layer "B.Cu") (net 22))
 (segment (start 158.644 75.4581) (end 159.8696 75.4581) (width 0.25) (layer "B.Cu") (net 22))
 (segment (start 166.106 80.1067) (end 167.169 80.1067) (width 0.25) (layer "B.Cu") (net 22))
 (segment (start 159.8696 75.4581) (end 159.9278 75.3999) (width 0.25) (layer "B.Cu") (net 22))
 (segment (start 168.4002 93.5473) (end 165.5088 96.4387) (width 0.25) (layer "B.Cu") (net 22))
 (segment (start 168.4002 81.3379) (end 168.4002 93.5473) (width 0.25) (layer "B.Cu") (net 22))
 (segment (start 167.169 80.1067) (end 168.4002 81.3379) (width 0.25) (layer "B.Cu") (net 22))
 (segment (start 155.155 76.84) (end 155.8763 76.84) (width 0.25) (layer "B.Cu") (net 22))
 (segment (start 161.3992 75.3999) (end 166.106 80.1067) (width 0.25) (layer "B.Cu") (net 22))
 (segment (start 158.5646 75.3787) (end 158.644 75.4581) (width 0.25) (layer "B.Cu") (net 22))
 (segment (start 157.3376 75.3787) (end 158.5646 75.3787) (width 0.25) (layer "B.Cu") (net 22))
 (segment (start 151.3452 95.4348) (end 149.16 97.62) (width 0.25) (layer "F.Cu") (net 19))
 (segment (start 168.2006 95.61) (end 168.0254 95.4348) (width 0.25) (layer "F.Cu") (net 19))
 (segment (start 168.0254 95.4348) (end 151.3452 95.4348) (width 0.25) (layer "F.Cu") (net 19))
 (via (at 168.2006 95.61) (size 0.6) (drill 0.3) (layers "F.Cu" "B.Cu") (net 19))
 (segment (start 159.31 74) (end 161.0624 74) (width 0.25) (layer "B.Cu") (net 19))
 (segment (start 169.1534 94.6572) (end 168.2006 95.61) (width 0.25) (layer "B.Cu") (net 19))
 (segment (start 161.0624 74) (end 166.4174 79.355) (width 0.25) (layer "B.Cu") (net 19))
 (segment (start 169.1534 81.0279) (end 169.1534 94.6572) (width 0.25) (layer "B.Cu") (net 19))
 (segment (start 166.4174 79.355) (end 167.4805 79.355) (width 0.25) (layer "B.Cu") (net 19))
 (segment (start 167.4805 79.355) (end 169.1534 81.0279) (width 0.25) (layer "B.Cu") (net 19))
 (segment (start 131.7002 76.5011) (end 131.7002 74.3497) (width 0.25) (layer "F.Cu") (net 12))
 (segment (start 144.08 82.38) (end 140.9088 79.2088) (width 0.25) (layer "F.Cu") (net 12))
 (segment (start 135.8749 70.175) (end 153.8671 70.175) (width 0.25) (layer "F.Cu") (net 12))
 (segment (start 134.4079 79.2088) (end 131.7002 76.5011) (width 0.25) (layer "F.Cu") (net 12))
 (segment (start 140.9088 79.2088) (end 134.4079 79.2088) (width 0.25) (layer "F.Cu") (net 12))
 (segment (start 131.7002 74.3497) (end 135.8749 70.175) (width 0.25) (layer "F.Cu") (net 12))
 (via (at 153.8671 70.175) (size 0.6) (drill 0.3) (layers "F.Cu" "B.Cu") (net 12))
 (segment (start 153.8671 70.175) (end 153.77 70.2721) (width 0.25) (layer "B.Cu") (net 12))
 (segment (start 153.77 70.2721) (end 153.77 74) (width 0.25) (layer "B.Cu") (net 12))
 (segment (start 157.747 91.0723) (end 137.9277 91.0723) (width 0.25) (layer "F.Cu") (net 6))
 (segment (start 159.32 92.6453) (end 157.747 91.0723) (width 0.25) (layer "F.Cu") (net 6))
 (segment (start 137.9277 91.0723) (end 134 95) (width 0.25) (layer "F.Cu") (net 6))
 (via (at 159.32 92.6453) (size 0.6) (drill 0.3) (layers "F.Cu" "B.Cu") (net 6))
 (segment (start 159.32 82.38) (end 159.32 83.8067) (width 0.25) (layer "B.Cu") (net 6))
 (segment (start 159.32 92.6453) (end 159.32 83.8067) (width 0.25) (layer "B.Cu") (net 6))
 (segment (start 166.94 82.38) (end 159.8234 89.4966) (width 0.25) (layer "F.Cu") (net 2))
 (segment (start 135.5034 89.4966) (end 134 91) (width 0.25) (layer "F.Cu") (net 2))
 (segment (start 159.8234 89.4966) (end 135.5034 89.4966) (width 0.25) (layer "F.Cu") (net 2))
 (segment (start 147.7059 83.8341) (end 138.4291 83.8341) (width 0.25) (layer "F.Cu") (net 10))
 (segment (start 136.3777 81.7827) (end 136.3777 81.2858) (width 0.25) (layer "F.Cu") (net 10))
 (segment (start 149.16 82.38) (end 147.7059 83.8341) (width 0.25) (layer "F.Cu") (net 10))
 (segment (start 138.4291 83.8341) (end 136.3777 81.7827) (width 0.25) (layer "F.Cu") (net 10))
 (via (at 136.3777 81.2858) (size 0.6) (drill 0.3) (layers "F.Cu" "B.Cu") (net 10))
 (segment (start 136.3777 81.2858) (end 136.3777 78.2435) (width 0.25) (layer "B.Cu") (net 10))
 (segment (start 149.5733 72.5733) (end 151 74) (width 0.25) (layer "B.Cu") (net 10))
 (segment (start 142.0479 72.5733) (end 149.5733 72.5733) (width 0.25) (layer "B.Cu") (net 10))
 (segment (start 136.3777 78.2435) (end 142.0479 72.5733) (width 0.25) (layer "B.Cu") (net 10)))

